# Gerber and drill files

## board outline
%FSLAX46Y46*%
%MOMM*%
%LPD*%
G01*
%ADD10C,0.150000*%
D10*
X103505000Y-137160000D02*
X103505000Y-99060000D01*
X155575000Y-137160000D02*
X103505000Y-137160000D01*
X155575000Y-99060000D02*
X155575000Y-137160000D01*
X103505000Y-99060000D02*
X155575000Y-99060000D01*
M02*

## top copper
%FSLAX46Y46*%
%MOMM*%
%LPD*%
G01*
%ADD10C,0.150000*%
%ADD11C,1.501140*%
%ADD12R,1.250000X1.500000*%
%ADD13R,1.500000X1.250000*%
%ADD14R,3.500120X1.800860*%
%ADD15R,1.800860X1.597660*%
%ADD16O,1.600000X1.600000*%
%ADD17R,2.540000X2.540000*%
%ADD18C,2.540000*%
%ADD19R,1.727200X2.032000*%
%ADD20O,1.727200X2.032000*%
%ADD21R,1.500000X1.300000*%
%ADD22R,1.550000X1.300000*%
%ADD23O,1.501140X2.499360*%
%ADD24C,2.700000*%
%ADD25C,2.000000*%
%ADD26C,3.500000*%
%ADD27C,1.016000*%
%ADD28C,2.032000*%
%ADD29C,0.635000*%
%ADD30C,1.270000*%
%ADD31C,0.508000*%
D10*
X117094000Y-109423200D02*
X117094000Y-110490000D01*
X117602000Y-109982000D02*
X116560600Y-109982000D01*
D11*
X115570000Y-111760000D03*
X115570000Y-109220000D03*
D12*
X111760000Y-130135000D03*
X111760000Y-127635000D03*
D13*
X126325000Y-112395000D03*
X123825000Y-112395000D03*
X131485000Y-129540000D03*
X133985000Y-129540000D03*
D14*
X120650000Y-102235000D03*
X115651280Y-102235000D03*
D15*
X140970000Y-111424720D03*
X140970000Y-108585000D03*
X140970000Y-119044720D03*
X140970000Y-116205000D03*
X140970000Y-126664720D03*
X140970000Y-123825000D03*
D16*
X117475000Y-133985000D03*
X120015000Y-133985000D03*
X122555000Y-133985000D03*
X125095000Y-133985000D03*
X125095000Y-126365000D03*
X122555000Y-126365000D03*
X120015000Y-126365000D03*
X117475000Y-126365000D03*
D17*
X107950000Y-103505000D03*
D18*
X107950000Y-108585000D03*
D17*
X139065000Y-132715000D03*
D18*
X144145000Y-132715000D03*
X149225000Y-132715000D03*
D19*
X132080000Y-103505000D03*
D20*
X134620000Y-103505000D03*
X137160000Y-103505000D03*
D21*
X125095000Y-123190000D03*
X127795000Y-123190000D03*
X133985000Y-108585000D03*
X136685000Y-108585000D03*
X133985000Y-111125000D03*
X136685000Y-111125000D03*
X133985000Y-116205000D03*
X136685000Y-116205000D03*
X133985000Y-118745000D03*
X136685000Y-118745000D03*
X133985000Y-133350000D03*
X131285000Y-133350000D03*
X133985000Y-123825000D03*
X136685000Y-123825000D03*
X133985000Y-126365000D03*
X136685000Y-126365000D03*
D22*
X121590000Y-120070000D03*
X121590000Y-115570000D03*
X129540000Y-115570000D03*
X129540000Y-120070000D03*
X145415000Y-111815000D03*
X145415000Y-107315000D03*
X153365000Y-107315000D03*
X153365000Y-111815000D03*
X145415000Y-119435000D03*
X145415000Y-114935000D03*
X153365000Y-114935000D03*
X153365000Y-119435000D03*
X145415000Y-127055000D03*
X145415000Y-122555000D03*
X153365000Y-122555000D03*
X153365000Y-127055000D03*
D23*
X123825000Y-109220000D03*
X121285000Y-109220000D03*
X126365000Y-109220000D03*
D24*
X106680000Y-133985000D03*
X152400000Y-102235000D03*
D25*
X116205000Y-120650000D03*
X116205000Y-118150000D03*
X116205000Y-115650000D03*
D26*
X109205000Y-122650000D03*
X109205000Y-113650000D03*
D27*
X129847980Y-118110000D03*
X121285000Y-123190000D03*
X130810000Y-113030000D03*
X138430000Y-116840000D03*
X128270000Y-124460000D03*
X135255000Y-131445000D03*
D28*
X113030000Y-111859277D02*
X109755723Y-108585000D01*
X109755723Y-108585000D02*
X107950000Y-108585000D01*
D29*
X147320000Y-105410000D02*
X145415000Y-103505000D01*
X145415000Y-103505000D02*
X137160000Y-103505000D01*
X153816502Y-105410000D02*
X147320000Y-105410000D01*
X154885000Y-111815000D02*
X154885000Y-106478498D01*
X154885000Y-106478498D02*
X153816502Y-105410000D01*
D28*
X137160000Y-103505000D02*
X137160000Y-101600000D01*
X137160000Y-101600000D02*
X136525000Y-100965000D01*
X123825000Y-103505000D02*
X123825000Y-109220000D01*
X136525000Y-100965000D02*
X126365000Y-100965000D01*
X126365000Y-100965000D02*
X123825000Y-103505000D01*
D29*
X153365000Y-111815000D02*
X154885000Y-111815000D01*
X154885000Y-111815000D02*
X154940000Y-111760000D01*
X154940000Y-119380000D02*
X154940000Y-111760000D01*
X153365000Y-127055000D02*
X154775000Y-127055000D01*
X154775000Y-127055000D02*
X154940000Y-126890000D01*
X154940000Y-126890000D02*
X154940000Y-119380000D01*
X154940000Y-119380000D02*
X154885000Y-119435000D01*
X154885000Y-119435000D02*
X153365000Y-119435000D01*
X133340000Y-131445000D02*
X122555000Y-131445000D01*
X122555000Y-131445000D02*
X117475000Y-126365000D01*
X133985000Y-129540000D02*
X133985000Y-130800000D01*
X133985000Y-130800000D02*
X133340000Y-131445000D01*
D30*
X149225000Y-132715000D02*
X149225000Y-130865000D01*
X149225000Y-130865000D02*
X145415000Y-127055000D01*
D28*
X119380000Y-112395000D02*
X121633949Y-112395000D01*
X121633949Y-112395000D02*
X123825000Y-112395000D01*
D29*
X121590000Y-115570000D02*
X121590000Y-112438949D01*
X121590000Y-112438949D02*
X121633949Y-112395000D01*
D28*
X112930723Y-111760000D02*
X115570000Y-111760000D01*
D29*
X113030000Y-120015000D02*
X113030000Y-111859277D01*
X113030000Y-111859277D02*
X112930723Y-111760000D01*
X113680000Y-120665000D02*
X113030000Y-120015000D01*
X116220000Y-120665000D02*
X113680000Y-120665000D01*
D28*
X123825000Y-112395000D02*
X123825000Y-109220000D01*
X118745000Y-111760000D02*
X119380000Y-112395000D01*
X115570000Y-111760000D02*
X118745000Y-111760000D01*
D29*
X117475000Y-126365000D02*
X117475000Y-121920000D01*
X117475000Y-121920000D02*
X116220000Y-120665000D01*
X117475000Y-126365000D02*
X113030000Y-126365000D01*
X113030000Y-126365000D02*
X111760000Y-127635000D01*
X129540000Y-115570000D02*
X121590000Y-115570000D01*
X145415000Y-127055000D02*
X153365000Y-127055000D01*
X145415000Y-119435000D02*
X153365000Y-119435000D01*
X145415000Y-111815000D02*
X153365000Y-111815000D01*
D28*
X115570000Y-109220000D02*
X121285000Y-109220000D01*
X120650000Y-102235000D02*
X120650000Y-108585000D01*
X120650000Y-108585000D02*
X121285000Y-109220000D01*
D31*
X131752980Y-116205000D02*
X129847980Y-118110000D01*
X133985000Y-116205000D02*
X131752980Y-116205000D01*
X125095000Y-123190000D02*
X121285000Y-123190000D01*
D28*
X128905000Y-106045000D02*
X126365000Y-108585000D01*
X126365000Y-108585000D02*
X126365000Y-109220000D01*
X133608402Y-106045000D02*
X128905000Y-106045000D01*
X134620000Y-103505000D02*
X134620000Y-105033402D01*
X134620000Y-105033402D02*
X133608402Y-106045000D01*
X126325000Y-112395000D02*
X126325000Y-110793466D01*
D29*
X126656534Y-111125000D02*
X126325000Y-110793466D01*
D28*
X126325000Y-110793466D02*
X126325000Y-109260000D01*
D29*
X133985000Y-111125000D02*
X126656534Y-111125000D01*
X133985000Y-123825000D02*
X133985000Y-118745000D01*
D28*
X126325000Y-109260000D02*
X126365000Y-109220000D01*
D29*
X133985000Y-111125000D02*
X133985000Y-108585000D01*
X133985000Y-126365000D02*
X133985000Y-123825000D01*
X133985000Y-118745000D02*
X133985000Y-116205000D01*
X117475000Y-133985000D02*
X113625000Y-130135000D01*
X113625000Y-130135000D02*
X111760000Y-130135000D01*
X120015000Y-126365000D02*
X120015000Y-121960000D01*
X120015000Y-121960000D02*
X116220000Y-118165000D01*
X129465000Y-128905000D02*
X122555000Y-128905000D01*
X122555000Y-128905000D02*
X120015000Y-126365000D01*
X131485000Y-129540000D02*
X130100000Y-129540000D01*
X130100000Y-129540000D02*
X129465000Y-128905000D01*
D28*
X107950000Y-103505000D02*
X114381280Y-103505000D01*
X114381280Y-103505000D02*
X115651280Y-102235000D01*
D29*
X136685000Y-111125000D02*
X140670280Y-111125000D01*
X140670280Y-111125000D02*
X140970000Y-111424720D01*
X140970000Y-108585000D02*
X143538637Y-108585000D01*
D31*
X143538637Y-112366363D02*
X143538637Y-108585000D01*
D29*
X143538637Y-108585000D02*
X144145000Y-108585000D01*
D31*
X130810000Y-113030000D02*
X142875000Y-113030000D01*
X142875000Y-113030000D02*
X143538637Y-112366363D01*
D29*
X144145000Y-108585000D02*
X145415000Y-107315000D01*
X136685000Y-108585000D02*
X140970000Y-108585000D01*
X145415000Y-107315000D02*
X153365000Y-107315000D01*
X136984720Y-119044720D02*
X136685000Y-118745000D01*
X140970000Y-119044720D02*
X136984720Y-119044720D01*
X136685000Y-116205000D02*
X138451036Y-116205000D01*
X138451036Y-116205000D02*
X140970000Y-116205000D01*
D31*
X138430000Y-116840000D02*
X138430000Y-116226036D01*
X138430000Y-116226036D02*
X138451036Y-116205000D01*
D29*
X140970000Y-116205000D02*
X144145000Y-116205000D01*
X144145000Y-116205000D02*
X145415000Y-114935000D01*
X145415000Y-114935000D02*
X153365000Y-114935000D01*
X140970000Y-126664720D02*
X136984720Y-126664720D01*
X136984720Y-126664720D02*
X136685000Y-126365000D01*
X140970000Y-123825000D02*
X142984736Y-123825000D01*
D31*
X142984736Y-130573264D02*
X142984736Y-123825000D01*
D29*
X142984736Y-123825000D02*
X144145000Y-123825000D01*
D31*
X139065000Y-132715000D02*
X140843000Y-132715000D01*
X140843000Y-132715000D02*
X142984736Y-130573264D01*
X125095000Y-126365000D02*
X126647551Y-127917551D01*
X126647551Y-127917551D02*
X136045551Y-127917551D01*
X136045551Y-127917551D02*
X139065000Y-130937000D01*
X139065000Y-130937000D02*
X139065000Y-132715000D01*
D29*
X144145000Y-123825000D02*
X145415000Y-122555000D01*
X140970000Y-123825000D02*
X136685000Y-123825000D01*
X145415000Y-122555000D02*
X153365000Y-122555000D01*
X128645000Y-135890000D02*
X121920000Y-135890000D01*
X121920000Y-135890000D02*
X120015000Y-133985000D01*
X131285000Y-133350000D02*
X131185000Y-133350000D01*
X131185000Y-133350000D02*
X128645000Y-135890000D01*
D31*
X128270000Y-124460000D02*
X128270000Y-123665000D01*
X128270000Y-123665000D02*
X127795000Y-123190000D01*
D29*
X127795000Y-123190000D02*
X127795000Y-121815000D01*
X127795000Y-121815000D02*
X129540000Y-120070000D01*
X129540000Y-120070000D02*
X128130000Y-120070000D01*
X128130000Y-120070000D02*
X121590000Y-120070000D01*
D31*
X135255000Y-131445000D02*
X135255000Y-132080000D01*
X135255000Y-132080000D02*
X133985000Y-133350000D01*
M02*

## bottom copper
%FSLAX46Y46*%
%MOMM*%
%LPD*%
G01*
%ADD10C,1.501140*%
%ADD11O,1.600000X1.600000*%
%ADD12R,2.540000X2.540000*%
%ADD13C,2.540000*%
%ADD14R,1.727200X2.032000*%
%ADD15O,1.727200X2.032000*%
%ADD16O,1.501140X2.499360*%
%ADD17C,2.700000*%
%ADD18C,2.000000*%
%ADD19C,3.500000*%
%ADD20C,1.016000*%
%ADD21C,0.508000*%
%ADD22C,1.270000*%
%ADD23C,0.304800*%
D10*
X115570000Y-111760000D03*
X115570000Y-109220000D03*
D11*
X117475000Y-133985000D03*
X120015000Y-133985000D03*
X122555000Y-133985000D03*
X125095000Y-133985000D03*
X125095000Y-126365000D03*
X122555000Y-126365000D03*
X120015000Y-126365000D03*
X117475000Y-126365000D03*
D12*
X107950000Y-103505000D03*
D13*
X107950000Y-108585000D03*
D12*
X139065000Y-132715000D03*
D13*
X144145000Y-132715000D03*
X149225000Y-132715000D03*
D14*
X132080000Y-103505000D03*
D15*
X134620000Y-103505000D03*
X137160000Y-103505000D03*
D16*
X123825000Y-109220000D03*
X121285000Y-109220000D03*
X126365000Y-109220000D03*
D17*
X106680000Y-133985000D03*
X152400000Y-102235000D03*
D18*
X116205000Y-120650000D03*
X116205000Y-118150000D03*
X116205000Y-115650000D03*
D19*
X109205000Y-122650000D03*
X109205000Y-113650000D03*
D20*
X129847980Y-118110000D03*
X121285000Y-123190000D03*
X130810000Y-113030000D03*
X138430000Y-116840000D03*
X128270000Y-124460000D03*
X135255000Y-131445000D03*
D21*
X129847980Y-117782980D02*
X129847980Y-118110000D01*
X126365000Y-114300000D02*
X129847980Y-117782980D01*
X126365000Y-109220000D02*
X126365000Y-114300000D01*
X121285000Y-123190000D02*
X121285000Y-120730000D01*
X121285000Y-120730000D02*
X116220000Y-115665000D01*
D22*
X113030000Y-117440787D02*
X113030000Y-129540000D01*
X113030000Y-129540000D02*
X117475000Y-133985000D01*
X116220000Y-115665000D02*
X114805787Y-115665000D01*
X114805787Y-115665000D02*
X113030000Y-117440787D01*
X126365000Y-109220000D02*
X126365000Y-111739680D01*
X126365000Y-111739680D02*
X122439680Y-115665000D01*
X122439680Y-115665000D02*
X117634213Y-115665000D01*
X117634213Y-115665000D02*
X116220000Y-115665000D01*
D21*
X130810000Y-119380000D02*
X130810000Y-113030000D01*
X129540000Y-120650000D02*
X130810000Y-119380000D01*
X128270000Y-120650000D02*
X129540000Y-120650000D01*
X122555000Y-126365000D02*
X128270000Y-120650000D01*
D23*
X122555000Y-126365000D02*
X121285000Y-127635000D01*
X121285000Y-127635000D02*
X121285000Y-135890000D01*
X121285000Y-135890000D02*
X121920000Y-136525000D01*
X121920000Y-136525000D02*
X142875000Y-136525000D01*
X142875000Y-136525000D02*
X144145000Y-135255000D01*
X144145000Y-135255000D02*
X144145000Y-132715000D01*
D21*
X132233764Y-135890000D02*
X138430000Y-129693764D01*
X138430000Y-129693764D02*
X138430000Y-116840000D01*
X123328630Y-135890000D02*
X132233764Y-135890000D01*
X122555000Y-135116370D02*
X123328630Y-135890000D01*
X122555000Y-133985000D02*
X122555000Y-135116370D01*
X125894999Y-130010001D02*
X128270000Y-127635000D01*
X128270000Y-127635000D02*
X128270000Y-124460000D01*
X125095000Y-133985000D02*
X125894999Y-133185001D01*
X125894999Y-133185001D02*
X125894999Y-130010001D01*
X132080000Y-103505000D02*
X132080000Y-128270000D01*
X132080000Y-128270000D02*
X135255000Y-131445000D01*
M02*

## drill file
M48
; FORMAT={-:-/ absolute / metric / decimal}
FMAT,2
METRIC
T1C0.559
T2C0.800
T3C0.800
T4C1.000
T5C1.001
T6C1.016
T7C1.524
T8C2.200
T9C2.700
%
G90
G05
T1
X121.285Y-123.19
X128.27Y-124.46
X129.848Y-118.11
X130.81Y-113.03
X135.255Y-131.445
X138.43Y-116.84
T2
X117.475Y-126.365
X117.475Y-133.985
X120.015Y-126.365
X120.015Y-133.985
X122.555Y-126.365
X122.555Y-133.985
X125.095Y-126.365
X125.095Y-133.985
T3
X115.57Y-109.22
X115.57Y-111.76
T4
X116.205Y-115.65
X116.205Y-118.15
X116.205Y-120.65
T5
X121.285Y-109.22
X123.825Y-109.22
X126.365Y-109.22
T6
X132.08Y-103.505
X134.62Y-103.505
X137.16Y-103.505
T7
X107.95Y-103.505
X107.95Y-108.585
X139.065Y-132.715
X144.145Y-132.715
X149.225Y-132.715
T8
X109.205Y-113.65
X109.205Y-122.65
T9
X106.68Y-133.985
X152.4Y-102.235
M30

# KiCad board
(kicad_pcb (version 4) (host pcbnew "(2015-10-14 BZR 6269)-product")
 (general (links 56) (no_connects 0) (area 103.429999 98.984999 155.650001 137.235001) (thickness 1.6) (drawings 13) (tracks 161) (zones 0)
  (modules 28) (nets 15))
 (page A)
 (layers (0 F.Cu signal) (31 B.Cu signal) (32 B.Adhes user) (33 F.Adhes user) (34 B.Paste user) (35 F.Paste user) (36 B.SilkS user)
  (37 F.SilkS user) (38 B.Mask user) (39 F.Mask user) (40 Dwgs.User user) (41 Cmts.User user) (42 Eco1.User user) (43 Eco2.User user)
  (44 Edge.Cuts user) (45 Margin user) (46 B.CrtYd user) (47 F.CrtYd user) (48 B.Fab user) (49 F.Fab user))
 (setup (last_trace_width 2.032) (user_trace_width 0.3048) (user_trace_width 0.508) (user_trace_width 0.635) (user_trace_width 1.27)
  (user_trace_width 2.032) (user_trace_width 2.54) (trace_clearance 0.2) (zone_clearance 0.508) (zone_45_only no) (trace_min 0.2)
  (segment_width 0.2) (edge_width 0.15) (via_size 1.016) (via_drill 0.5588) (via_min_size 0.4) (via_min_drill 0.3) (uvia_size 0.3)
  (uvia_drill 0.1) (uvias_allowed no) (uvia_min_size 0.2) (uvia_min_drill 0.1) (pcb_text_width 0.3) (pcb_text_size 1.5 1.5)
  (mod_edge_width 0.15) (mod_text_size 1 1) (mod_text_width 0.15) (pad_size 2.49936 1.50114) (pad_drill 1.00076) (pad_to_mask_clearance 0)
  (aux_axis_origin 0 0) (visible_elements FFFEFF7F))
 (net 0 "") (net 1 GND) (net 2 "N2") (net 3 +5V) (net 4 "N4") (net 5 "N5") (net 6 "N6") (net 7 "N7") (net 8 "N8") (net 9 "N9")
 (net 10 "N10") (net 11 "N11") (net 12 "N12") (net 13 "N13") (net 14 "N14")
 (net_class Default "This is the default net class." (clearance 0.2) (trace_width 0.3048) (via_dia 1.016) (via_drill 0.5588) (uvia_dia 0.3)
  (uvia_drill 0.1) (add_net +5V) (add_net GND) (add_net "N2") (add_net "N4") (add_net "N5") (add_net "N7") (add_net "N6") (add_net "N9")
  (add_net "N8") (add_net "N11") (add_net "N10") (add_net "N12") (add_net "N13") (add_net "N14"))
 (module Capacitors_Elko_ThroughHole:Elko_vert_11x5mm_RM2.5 (layer F.Cu) (at 115.57 109.22 270)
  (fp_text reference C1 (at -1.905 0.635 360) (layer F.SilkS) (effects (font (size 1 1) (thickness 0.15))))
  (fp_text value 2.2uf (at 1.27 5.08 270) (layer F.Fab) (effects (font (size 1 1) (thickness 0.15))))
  (fp_line (start 0.2032 -1.524) (end 1.27 -1.524) (layer F.Cu) (width 0.15))
  (fp_line (start 0.762 -2.032) (end 0.762 -0.9906) (layer F.Cu) (width 0.15))
  (pad 2 thru_hole circle (at 2.54 0 270) (size 1.50114 1.50114) (drill 0.8001) (layers *.Cu *.Mask F.SilkS) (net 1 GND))
  (pad 1 thru_hole circle (at 0 0 270) (size 1.50114 1.50114) (drill 0.8001) (layers *.Cu *.Mask F.SilkS) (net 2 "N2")))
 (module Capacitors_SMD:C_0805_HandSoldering (layer F.Cu) (at 111.76 128.885 90)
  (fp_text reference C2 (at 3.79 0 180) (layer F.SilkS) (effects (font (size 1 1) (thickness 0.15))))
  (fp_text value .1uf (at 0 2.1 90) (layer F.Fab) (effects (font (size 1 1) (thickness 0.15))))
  (pad 1 smd rect (at -1.25 0 90) (size 1.5 1.25) (layers F.Cu F.Paste F.Mask) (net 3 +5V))
  (pad 2 smd rect (at 1.25 0 90) (size 1.5 1.25) (layers F.Cu F.Paste F.Mask) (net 1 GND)))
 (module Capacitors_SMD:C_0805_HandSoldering (layer F.Cu) (at 125.075 112.395 180)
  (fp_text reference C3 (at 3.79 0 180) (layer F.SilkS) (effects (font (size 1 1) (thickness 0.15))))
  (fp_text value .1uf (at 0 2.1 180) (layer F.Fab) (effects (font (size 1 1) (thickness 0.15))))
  (pad 1 smd rect (at -1.25 0 180) (size 1.5 1.25) (layers F.Cu F.Paste F.Mask) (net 3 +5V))
  (pad 2 smd rect (at 1.25 0 180) (size 1.5 1.25) (layers F.Cu F.Paste F.Mask) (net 1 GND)))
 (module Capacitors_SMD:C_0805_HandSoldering (layer F.Cu) (at 132.735 129.54)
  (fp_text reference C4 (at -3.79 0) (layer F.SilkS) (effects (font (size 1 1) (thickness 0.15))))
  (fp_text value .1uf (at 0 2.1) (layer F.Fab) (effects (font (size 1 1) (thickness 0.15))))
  (pad 1 smd rect (at -1.25 0) (size 1.5 1.25) (layers F.Cu F.Paste F.Mask) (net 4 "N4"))
  (pad 2 smd rect (at 1.25 0) (size 1.5 1.25) (layers F.Cu F.Paste F.Mask) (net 1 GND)))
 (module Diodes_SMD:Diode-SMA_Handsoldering (layer F.Cu) (at 118.15064 102.235 180)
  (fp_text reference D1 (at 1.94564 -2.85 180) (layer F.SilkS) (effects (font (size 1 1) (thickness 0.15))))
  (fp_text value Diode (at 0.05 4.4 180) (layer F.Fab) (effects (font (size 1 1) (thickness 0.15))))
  (pad 1 smd rect (at -2.49936 0 180) (size 3.50012 1.80086) (layers F.Cu F.Paste F.Mask) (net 2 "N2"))
  (pad 2 smd rect (at 2.49936 0 180) (size 3.50012 1.80086) (layers F.Cu F.Paste F.Mask) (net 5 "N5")))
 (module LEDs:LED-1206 (layer F.Cu) (at 140.97 110.00486 270)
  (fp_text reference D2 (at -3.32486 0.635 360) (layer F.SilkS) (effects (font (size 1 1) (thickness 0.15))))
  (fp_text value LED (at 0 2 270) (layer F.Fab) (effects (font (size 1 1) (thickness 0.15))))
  (pad 2 smd rect (at 1.41986 0 90) (size 1.59766 1.80086) (layers F.Cu F.Paste F.Mask) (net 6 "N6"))
  (pad 1 smd rect (at -1.41986 0 90) (size 1.59766 1.80086) (layers F.Cu F.Paste F.Mask) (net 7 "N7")))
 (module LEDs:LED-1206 (layer F.Cu) (at 140.97 117.62486 270)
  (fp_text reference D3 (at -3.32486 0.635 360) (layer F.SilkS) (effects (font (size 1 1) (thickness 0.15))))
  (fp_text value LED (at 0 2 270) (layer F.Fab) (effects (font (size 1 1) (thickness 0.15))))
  (pad 2 smd rect (at 1.41986 0 90) (size 1.59766 1.80086) (layers F.Cu F.Paste F.Mask) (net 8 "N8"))
  (pad 1 smd rect (at -1.41986 0 90) (size 1.59766 1.80086) (layers F.Cu F.Paste F.Mask) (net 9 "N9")))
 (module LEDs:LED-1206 (layer F.Cu) (at 140.97 125.24486 270)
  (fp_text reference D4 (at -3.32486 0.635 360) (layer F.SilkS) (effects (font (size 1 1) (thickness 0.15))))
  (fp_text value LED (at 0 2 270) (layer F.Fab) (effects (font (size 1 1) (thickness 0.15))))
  (pad 2 smd rect (at 1.41986 0 90) (size 1.59766 1.80086) (layers F.Cu F.Paste F.Mask) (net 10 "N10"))
  (pad 1 smd rect (at -1.41986 0 90) (size 1.59766 1.80086) (layers F.Cu F.Paste F.Mask) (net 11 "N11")))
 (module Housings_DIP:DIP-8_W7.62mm (layer F.Cu) (at 117.475 133.985 90)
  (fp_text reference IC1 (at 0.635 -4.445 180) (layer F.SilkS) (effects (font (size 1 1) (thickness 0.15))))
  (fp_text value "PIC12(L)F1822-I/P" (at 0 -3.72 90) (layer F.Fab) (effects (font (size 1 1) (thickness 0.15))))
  (pad 1 thru_hole oval (at 0 0 90) (size 1.6 1.6) (drill 0.8) (layers *.Cu *.Mask F.SilkS) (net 3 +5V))
  (pad 2 thru_hole oval (at 0 2.54 90) (size 1.6 1.6) (drill 0.8) (layers *.Cu *.Mask F.SilkS) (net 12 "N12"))
  (pad 3 thru_hole oval (at 0 5.08 90) (size 1.6 1.6) (drill 0.8) (layers *.Cu *.Mask F.SilkS) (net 9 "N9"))
  (pad 4 thru_hole oval (at 0 7.62 90) (size 1.6 1.6) (drill 0.8) (layers *.Cu *.Mask F.SilkS) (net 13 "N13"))
  (pad 5 thru_hole oval (at 7.62 7.62 90) (size 1.6 1.6) (drill 0.8) (layers *.Cu *.Mask F.SilkS) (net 11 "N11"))
  (pad 6 thru_hole oval (at 7.62 5.08 90) (size 1.6 1.6) (drill 0.8) (layers *.Cu *.Mask F.SilkS) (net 7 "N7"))
  (pad 7 thru_hole oval (at 7.62 2.54 90) (size 1.6 1.6) (drill 0.8) (layers *.Cu *.Mask F.SilkS) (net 4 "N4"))
  (pad 8 thru_hole oval (at 7.62 0 90) (size 1.6 1.6) (drill 0.8) (layers *.Cu *.Mask F.SilkS) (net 1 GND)))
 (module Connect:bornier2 (layer F.Cu) (at 107.95 106.045 270)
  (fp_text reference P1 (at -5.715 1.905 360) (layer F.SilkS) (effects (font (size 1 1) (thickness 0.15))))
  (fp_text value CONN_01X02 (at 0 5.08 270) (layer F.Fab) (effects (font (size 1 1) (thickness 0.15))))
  (pad 1 thru_hole rect (at -2.54 0 270) (size 2.54 2.54) (drill 1.524) (layers *.Cu *.Mask F.SilkS) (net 5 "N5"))
  (pad 2 thru_hole circle (at 2.54 0 270) (size 2.54 2.54) (drill 1.524) (layers *.Cu *.Mask F.SilkS) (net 1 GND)))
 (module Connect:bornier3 (layer F.Cu) (at 144.145 132.715)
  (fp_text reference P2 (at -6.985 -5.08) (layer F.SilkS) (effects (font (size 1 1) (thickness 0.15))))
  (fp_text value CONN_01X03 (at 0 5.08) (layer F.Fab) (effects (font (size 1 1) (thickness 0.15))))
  (pad 1 thru_hole rect (at -5.08 0) (size 2.54 2.54) (drill 1.524) (layers *.Cu *.Mask F.SilkS) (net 11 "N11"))
  (pad 2 thru_hole circle (at 0 0) (size 2.54 2.54) (drill 1.524) (layers *.Cu *.Mask F.SilkS) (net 7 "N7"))
  (pad 3 thru_hole circle (at 5.08 0) (size 2.54 2.54) (drill 1.524) (layers *.Cu *.Mask F.SilkS) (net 1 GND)))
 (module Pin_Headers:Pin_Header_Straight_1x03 (layer F.Cu) (at 132.08 103.505 90)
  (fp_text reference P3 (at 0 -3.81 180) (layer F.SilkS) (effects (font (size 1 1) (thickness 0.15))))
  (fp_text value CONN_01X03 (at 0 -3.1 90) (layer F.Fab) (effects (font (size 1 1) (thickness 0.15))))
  (pad 1 thru_hole rect (at 0 0 90) (size 2.032 1.7272) (drill 1.016) (layers *.Cu *.Mask F.SilkS) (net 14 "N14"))
  (pad 2 thru_hole oval (at 0 2.54 90) (size 2.032 1.7272) (drill 1.016) (layers *.Cu *.Mask F.SilkS) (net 3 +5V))
  (pad 3 thru_hole oval (at 0 5.08 90) (size 2.032 1.7272) (drill 1.016) (layers *.Cu *.Mask F.SilkS) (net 1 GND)))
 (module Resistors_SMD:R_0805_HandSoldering (layer F.Cu) (at 126.445 123.19)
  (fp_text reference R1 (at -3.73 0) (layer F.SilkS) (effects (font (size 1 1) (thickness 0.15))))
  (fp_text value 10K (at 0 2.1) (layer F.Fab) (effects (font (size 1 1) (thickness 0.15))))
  (pad 1 smd rect (at -1.35 0) (size 1.5 1.3) (layers F.Cu F.Paste F.Mask) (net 3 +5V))
  (pad 2 smd rect (at 1.35 0) (size 1.5 1.3) (layers F.Cu F.Paste F.Mask) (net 13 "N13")))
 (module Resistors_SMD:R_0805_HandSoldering (layer F.Cu) (at 135.335 108.585)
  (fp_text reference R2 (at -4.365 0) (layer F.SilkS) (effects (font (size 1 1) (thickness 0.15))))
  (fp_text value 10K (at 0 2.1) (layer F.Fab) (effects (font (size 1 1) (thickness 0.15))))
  (pad 1 smd rect (at -1.35 0) (size 1.5 1.3) (layers F.Cu F.Paste F.Mask) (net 3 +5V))
  (pad 2 smd rect (at 1.35 0) (size 1.5 1.3) (layers F.Cu F.Paste F.Mask) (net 7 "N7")))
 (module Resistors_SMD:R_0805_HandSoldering (layer F.Cu) (at 135.335 111.125)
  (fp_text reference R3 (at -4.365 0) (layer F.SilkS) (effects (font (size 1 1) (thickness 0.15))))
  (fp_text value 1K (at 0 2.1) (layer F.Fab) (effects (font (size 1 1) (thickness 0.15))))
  (pad 1 smd rect (at -1.35 0) (size 1.5 1.3) (layers F.Cu F.Paste F.Mask) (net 3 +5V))
  (pad 2 smd rect (at 1.35 0) (size 1.5 1.3) (layers F.Cu F.Paste F.Mask) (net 6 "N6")))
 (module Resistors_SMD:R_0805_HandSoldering (layer F.Cu) (at 135.335 116.205)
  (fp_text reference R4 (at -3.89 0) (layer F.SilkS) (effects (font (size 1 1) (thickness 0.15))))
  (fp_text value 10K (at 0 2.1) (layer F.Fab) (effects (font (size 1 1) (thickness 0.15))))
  (pad 1 smd rect (at -1.35 0) (size 1.5 1.3) (layers F.Cu F.Paste F.Mask) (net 3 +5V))
  (pad 2 smd rect (at 1.35 0) (size 1.5 1.3) (layers F.Cu F.Paste F.Mask) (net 9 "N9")))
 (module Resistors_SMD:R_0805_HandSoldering (layer F.Cu) (at 135.335 118.745)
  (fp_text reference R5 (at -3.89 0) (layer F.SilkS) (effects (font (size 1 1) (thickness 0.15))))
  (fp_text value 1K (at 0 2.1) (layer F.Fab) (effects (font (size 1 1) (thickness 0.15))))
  (pad 1 smd rect (at -1.35 0) (size 1.5 1.3) (layers F.Cu F.Paste F.Mask) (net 3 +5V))
  (pad 2 smd rect (at 1.35 0) (size 1.5 1.3) (layers F.Cu F.Paste F.Mask) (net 8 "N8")))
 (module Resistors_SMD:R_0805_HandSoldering (layer F.Cu) (at 132.635 133.35 180)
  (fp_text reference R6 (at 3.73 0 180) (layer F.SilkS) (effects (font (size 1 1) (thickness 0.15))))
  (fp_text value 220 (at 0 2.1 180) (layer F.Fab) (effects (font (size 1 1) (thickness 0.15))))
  (pad 1 smd rect (at -1.35 0 180) (size 1.5 1.3) (layers F.Cu F.Paste F.Mask) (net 14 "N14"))
  (pad 2 smd rect (at 1.35 0 180) (size 1.5 1.3) (layers F.Cu F.Paste F.Mask) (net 12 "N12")))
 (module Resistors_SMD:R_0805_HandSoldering (layer F.Cu) (at 135.335 123.825)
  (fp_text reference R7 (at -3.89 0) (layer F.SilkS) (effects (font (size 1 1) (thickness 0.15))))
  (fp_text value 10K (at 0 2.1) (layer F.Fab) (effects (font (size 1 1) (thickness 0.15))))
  (pad 1 smd rect (at -1.35 0) (size 1.5 1.3) (layers F.Cu F.Paste F.Mask) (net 3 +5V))
  (pad 2 smd rect (at 1.35 0) (size 1.5 1.3) (layers F.Cu F.Paste F.Mask) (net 11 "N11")))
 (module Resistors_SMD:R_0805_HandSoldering (layer F.Cu) (at 135.335 126.365)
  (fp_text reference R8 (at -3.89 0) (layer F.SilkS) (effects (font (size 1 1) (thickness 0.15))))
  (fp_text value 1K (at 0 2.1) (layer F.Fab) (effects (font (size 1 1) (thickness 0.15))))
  (pad 1 smd rect (at -1.35 0) (size 1.5 1.3) (layers F.Cu F.Paste F.Mask) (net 3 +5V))
  (pad 2 smd rect (at 1.35 0) (size 1.5 1.3) (layers F.Cu F.Paste F.Mask) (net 10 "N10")))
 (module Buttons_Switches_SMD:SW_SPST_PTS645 (layer F.Cu) (at 125.565 117.82)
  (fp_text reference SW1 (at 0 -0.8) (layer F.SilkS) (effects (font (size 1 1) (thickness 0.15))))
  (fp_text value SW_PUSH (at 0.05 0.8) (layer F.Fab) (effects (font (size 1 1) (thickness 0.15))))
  (pad 2 smd rect (at -3.975 2.25) (size 1.55 1.3) (layers F.Cu F.Paste F.Mask) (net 13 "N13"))
  (pad 1 smd rect (at -3.975 -2.25) (size 1.55 1.3) (layers F.Cu F.Paste F.Mask) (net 1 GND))
  (pad 1 smd rect (at 3.975 -2.25) (size 1.55 1.3) (layers F.Cu F.Paste F.Mask) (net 1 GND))
  (pad 2 smd rect (at 3.975 2.25) (size 1.55 1.3) (layers F.Cu F.Paste F.Mask) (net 13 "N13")))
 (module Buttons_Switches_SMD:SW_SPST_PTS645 (layer F.Cu) (at 149.39 109.565)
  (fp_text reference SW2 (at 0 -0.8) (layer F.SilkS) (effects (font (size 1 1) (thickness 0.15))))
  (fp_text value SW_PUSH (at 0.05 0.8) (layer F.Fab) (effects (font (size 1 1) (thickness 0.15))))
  (pad 2 smd rect (at -3.975 2.25) (size 1.55 1.3) (layers F.Cu F.Paste F.Mask) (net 1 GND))
  (pad 1 smd rect (at -3.975 -2.25) (size 1.55 1.3) (layers F.Cu F.Paste F.Mask) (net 7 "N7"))
  (pad 1 smd rect (at 3.975 -2.25) (size 1.55 1.3) (layers F.Cu F.Paste F.Mask) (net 7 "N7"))
  (pad 2 smd rect (at 3.975 2.25) (size 1.55 1.3) (layers F.Cu F.Paste F.Mask) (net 1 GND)))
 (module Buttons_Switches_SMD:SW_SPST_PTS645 (layer F.Cu) (at 149.39 117.185)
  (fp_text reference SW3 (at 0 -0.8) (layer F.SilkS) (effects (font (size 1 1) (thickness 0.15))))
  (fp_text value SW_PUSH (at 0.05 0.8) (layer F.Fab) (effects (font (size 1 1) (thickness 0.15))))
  (pad 2 smd rect (at -3.975 2.25) (size 1.55 1.3) (layers F.Cu F.Paste F.Mask) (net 1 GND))
  (pad 1 smd rect (at -3.975 -2.25) (size 1.55 1.3) (layers F.Cu F.Paste F.Mask) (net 9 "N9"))
  (pad 1 smd rect (at 3.975 -2.25) (size 1.55 1.3) (layers F.Cu F.Paste F.Mask) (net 9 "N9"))
  (pad 2 smd rect (at 3.975 2.25) (size 1.55 1.3) (layers F.Cu F.Paste F.Mask) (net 1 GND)))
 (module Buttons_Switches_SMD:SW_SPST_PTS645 (layer F.Cu) (at 149.39 124.805)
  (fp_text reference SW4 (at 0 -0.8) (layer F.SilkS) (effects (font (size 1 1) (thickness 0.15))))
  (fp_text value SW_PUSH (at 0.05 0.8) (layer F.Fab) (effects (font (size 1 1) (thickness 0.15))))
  (pad 2 smd rect (at -3.975 2.25) (size 1.55 1.3) (layers F.Cu F.Paste F.Mask) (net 1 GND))
  (pad 1 smd rect (at -3.975 -2.25) (size 1.55 1.3) (layers F.Cu F.Paste F.Mask) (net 11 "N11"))
  (pad 1 smd rect (at 3.975 -2.25) (size 1.55 1.3) (layers F.Cu F.Paste F.Mask) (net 11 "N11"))
  (pad 2 smd rect (at 3.975 2.25) (size 1.55 1.3) (layers F.Cu F.Paste F.Mask) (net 1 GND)))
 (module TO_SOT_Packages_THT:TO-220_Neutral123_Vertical (layer F.Cu) (at 123.825 109.22)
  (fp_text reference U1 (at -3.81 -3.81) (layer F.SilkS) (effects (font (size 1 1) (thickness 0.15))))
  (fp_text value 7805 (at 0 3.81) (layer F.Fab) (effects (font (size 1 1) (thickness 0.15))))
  (pad GND thru_hole oval (at 0 0 90) (size 2.49936 1.50114) (drill 1.00076) (layers *.Cu *.Mask F.SilkS) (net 1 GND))
  (pad VI thru_hole oval (at -2.54 0 90) (size 2.49936 1.50114) (drill 1.00076) (layers *.Cu *.Mask F.SilkS) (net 2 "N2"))
  (pad VO thru_hole oval (at 2.54 0 90) (size 2.49936 1.50114) (drill 1.00076) (layers *.Cu *.Mask F.SilkS) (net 3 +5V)))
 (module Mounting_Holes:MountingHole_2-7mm (layer F.Cu) (at 106.68 133.985)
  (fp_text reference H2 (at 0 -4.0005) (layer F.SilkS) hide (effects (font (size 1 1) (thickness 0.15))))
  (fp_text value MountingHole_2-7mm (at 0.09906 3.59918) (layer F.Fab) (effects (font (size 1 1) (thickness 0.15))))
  (pad 1 thru_hole circle (at 0 0) (size 2.7 2.7) (drill 2.7) (layers)))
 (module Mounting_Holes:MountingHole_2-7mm (layer F.Cu) (at 152.4 102.235)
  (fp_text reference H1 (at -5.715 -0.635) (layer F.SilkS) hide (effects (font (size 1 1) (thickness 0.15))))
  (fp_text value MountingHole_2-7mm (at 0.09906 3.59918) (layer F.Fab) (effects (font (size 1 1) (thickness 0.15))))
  (pad 1 thru_hole circle (at 0 0) (size 2.7 2.7) (drill 2.7) (layers)))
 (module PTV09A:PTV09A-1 (layer F.Cu) (at 116.205 118.15 90)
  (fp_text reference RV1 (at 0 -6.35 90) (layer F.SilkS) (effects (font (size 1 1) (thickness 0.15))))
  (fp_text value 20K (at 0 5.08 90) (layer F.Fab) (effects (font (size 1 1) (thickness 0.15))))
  (pad 1 thru_hole circle (at -2.5 0 90) (size 2 2) (drill 1) (layers *.Cu *.Mask F.SilkS) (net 1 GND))
  (pad 2 thru_hole circle (at 0 0 90) (size 2 2) (drill 1) (layers *.Cu *.Mask F.SilkS) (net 4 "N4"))
  (pad 3 thru_hole circle (at 2.5 0 90) (size 2 2) (drill 1) (layers *.Cu *.Mask F.SilkS) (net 3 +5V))
  (pad 4 thru_hole circle (at -4.5 -7 90) (size 3.5 3.5) (drill 2.2) (layers *.Cu *.Mask F.SilkS))
  (pad 4 thru_hole circle (at 4.5 -7 90) (size 3.5 3.5) (drill 2.2) (layers *.Cu *.Mask F.SilkS)))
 (gr_line (start 103.505 137.16) (end 103.505 99.06) (layer Edge.Cuts) (width 0.15))
 (gr_line (start 155.575 137.16) (end 103.505 137.16) (layer Edge.Cuts) (width 0.15))
 (gr_line (start 155.575 99.06) (end 155.575 137.16) (layer Edge.Cuts) (width 0.15))
 (gr_line (start 103.505 99.06) (end 155.575 99.06) (layer Edge.Cuts) (width 0.15))
 (segment (start 113.03 111.859277) (end 109.755723 108.585) (width 2.032) (layer F.Cu) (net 1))
 (segment (start 109.755723 108.585) (end 107.95 108.585) (width 2.032) (layer F.Cu) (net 1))
 (segment (start 147.32 105.41) (end 145.415 103.505) (width 0.635) (layer F.Cu) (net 1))
 (segment (start 145.415 103.505) (end 137.16 103.505) (width 0.635) (layer F.Cu) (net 1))
 (segment (start 153.816502 105.41) (end 147.32 105.41) (width 0.635) (layer F.Cu) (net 1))
 (segment (start 154.885 111.815) (end 154.885 106.478498) (width 0.635) (layer F.Cu) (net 1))
 (segment (start 154.885 106.478498) (end 153.816502 105.41) (width 0.635) (layer F.Cu) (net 1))
 (segment (start 137.16 103.505) (end 137.16 101.6) (width 2.032) (layer F.Cu) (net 1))
 (segment (start 137.16 101.6) (end 136.525 100.965) (width 2.032) (layer F.Cu) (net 1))
 (segment (start 123.825 103.505) (end 123.825 109.22) (width 2.032) (layer F.Cu) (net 1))
 (segment (start 136.525 100.965) (end 126.365 100.965) (width 2.032) (layer F.Cu) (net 1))
 (segment (start 126.365 100.965) (end 123.825 103.505) (width 2.032) (layer F.Cu) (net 1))
 (segment (start 153.365 111.815) (end 154.885 111.815) (width 0.635) (layer F.Cu) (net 1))
 (segment (start 154.885 111.815) (end 154.94 111.76) (width 0.635) (layer F.Cu) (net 1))
 (segment (start 154.94 119.38) (end 154.94 111.76) (width 0.635) (layer F.Cu) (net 1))
 (segment (start 153.365 127.055) (end 154.775 127.055) (width 0.635) (layer F.Cu) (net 1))
 (segment (start 154.775 127.055) (end 154.94 126.89) (width 0.635) (layer F.Cu) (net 1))
 (segment (start 154.94 126.89) (end 154.94 119.38) (width 0.635) (layer F.Cu) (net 1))
 (segment (start 154.94 119.38) (end 154.885 119.435) (width 0.635) (layer F.Cu) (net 1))
 (segment (start 154.885 119.435) (end 153.365 119.435) (width 0.635) (layer F.Cu) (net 1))
 (segment (start 133.34 131.445) (end 122.555 131.445) (width 0.635) (layer F.Cu) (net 1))
 (segment (start 122.555 131.445) (end 117.475 126.365) (width 0.635) (layer F.Cu) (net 1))
 (segment (start 133.985 129.54) (end 133.985 130.8) (width 0.635) (layer F.Cu) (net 1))
 (segment (start 133.985 130.8) (end 133.34 131.445) (width 0.635) (layer F.Cu) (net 1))
 (segment (start 149.225 132.715) (end 149.225 130.865) (width 1.27) (layer F.Cu) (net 1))
 (segment (start 149.225 130.865) (end 145.415 127.055) (width 1.27) (layer F.Cu) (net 1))
 (segment (start 119.38 112.395) (end 121.633949 112.395) (width 2.032) (layer F.Cu) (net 1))
 (segment (start 121.633949 112.395) (end 123.825 112.395) (width 2.032) (layer F.Cu) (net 1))
 (segment (start 121.59 115.57) (end 121.59 112.438949) (width 0.635) (layer F.Cu) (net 1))
 (segment (start 121.59 112.438949) (end 121.633949 112.395) (width 0.635) (layer F.Cu) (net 1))
 (segment (start 112.930723 111.76) (end 115.57 111.76) (width 2.032) (layer F.Cu) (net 1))
 (segment (start 113.03 120.015) (end 113.03 111.859277) (width 0.635) (layer F.Cu) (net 1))
 (segment (start 113.03 111.859277) (end 112.930723 111.76) (width 0.635) (layer F.Cu) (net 1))
 (segment (start 113.68 120.665) (end 113.03 120.015) (width 0.635) (layer F.Cu) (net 1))
 (segment (start 116.22 120.665) (end 113.68 120.665) (width 0.635) (layer F.Cu) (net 1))
 (segment (start 123.825 112.395) (end 123.825 109.22) (width 2.032) (layer F.Cu) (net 1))
 (segment (start 118.745 111.76) (end 119.38 112.395) (width 2.032) (layer F.Cu) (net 1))
 (segment (start 115.57 111.76) (end 118.745 111.76) (width 2.032) (layer F.Cu) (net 1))
 (segment (start 117.475 126.365) (end 117.475 121.92) (width 0.635) (layer F.Cu) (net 1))
 (segment (start 117.475 121.92) (end 116.22 120.665) (width 0.635) (layer F.Cu) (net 1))
 (segment (start 117.475 126.365) (end 113.03 126.365) (width 0.635) (layer F.Cu) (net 1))
 (segment (start 113.03 126.365) (end 111.76 127.635) (width 0.635) (layer F.Cu) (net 1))
 (segment (start 129.54 115.57) (end 121.59 115.57) (width 0.635) (layer F.Cu) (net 1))
 (segment (start 145.415 127.055) (end 153.365 127.055) (width 0.635) (layer F.Cu) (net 1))
 (segment (start 145.415 119.435) (end 153.365 119.435) (width 0.635) (layer F.Cu) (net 1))
 (segment (start 145.415 111.815) (end 153.365 111.815) (width 0.635) (layer F.Cu) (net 1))
 (segment (start 115.57 109.22) (end 121.285 109.22) (width 2.032) (layer F.Cu) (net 2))
 (segment (start 120.65 102.235) (end 120.65 108.585) (width 2.032) (layer F.Cu) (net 2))
 (segment (start 120.65 108.585) (end 121.285 109.22) (width 2.032) (layer F.Cu) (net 2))
 (segment (start 129.84798 117.78298) (end 129.84798 118.11) (width 0.508) (layer B.Cu) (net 3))
 (segment (start 126.365 114.3) (end 129.84798 117.78298) (width 0.508) (layer B.Cu) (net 3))
 (segment (start 126.365 109.22) (end 126.365 114.3) (width 0.508) (layer B.Cu) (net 3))
 (via (at 129.84798 118.11) (size 1.016) (drill 0.5588) (layers F.Cu B.Cu) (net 3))
 (segment (start 131.75298 116.205) (end 129.84798 118.11) (width 0.508) (layer F.Cu) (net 3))
 (segment (start 133.985 116.205) (end 131.75298 116.205) (width 0.508) (layer F.Cu) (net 3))
 (segment (start 121.285 123.19) (end 121.285 120.73) (width 0.508) (layer B.Cu) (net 3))
 (segment (start 121.285 120.73) (end 116.22 115.665) (width 0.508) (layer B.Cu) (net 3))
 (segment (start 125.095 123.19) (end 121.285 123.19) (width 0.508) (layer F.Cu) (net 3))
 (via (at 121.285 123.19) (size 1.016) (drill 0.5588) (layers F.Cu B.Cu) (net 3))
 (segment (start 128.905 106.045) (end 126.365 108.585) (width 2.032) (layer F.Cu) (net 3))
 (segment (start 126.365 108.585) (end 126.365 109.22) (width 2.032) (layer F.Cu) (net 3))
 (segment (start 133.608402 106.045) (end 128.905 106.045) (width 2.032) (layer F.Cu) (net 3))
 (segment (start 134.62 103.505) (end 134.62 105.033402) (width 2.032) (layer F.Cu) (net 3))
 (segment (start 134.62 105.033402) (end 133.608402 106.045) (width 2.032) (layer F.Cu) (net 3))
 (segment (start 113.03 117.440787) (end 113.03 129.54) (width 1.27) (layer B.Cu) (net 3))
 (segment (start 113.03 129.54) (end 117.475 133.985) (width 1.27) (layer B.Cu) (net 3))
 (segment (start 116.22 115.665) (end 114.805787 115.665) (width 1.27) (layer B.Cu) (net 3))
 (segment (start 114.805787 115.665) (end 113.03 117.440787) (width 1.27) (layer B.Cu) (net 3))
 (segment (start 126.365 109.22) (end 126.365 111.73968) (width 1.27) (layer B.Cu) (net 3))
 (segment (start 126.365 111.73968) (end 122.43968 115.665) (width 1.27) (layer B.Cu) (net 3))
 (segment (start 122.43968 115.665) (end 117.634213 115.665) (width 1.27) (layer B.Cu) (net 3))
 (segment (start 117.634213 115.665) (end 116.22 115.665) (width 1.27) (layer B.Cu) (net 3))
 (segment (start 126.325 112.395) (end 126.325 110.793466) (width 2.032) (layer F.Cu) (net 3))
 (segment (start 126.656534 111.125) (end 126.325 110.793466) (width 0.635) (layer F.Cu) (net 3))
 (segment (start 126.325 110.793466) (end 126.325 109.26) (width 2.032) (layer F.Cu) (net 3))
 (segment (start 133.985 111.125) (end 126.656534 111.125) (width 0.635) (layer F.Cu) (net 3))
 (segment (start 133.985 123.825) (end 133.985 118.745) (width 0.635) (layer F.Cu) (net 3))
 (segment (start 126.325 109.26) (end 126.365 109.22) (width 2.032) (layer F.Cu) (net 3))
 (segment (start 133.985 111.125) (end 133.985 108.585) (width 0.635) (layer F.Cu) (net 3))
 (segment (start 133.985 126.365) (end 133.985 123.825) (width 0.635) (layer F.Cu) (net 3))
 (segment (start 133.985 118.745) (end 133.985 116.205) (width 0.635) (layer F.Cu) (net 3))
 (segment (start 117.475 133.985) (end 113.625 130.135) (width 0.635) (layer F.Cu) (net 3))
 (segment (start 113.625 130.135) (end 111.76 130.135) (width 0.635) (layer F.Cu) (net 3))
 (segment (start 120.015 126.365) (end 120.015 121.96) (width 0.635) (layer F.Cu) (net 4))
 (segment (start 120.015 121.96) (end 116.22 118.165) (width 0.635) (layer F.Cu) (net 4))
 (segment (start 129.465 128.905) (end 122.555 128.905) (width 0.635) (layer F.Cu) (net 4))
 (segment (start 122.555 128.905) (end 120.015 126.365) (width 0.635) (layer F.Cu) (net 4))
 (segment (start 131.485 129.54) (end 130.1 129.54) (width 0.635) (layer F.Cu) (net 4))
 (segment (start 130.1 129.54) (end 129.465 128.905) (width 0.635) (layer F.Cu) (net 4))
 (segment (start 107.95 103.505) (end 114.38128 103.505) (width 2.032) (layer F.Cu) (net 5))
 (segment (start 114.38128 103.505) (end 115.65128 102.235) (width 2.032) (layer F.Cu) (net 5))
 (segment (start 136.685 111.125) (end 140.67028 111.125) (width 0.635) (layer F.Cu) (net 6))
 (segment (start 140.67028 111.125) (end 140.97 111.42472) (width 0.635) (layer F.Cu) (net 6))
 (segment (start 140.97 108.585) (end 143.538637 108.585) (width 0.635) (layer F.Cu) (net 7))
 (segment (start 143.538637 112.366363) (end 143.538637 108.585) (width 0.508) (layer F.Cu) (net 7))
 (segment (start 143.538637 108.585) (end 144.145 108.585) (width 0.635) (layer F.Cu) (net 7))
 (segment (start 130.81 113.03) (end 142.875 113.03) (width 0.508) (layer F.Cu) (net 7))
 (segment (start 142.875 113.03) (end 143.538637 112.366363) (width 0.508) (layer F.Cu) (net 7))
 (via (at 130.81 113.03) (size 1.016) (drill 0.5588) (layers F.Cu B.Cu) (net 7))
 (segment (start 130.81 119.38) (end 130.81 113.03) (width 0.508) (layer B.Cu) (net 7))
 (segment (start 129.54 120.65) (end 130.81 119.38) (width 0.508) (layer B.Cu) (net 7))
 (segment (start 128.27 120.65) (end 129.54 120.65) (width 0.508) (layer B.Cu) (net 7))
 (segment (start 122.555 126.365) (end 128.27 120.65) (width 0.508) (layer B.Cu) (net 7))
 (segment (start 122.555 126.365) (end 121.285 127.635) (width 0.3048) (layer B.Cu) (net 7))
 (segment (start 121.285 127.635) (end 121.285 135.89) (width 0.3048) (layer B.Cu) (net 7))
 (segment (start 121.285 135.89) (end 121.92 136.525) (width 0.3048) (layer B.Cu) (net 7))
 (segment (start 121.92 136.525) (end 142.875 136.525) (width 0.3048) (layer B.Cu) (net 7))
 (segment (start 142.875 136.525) (end 144.145 135.255) (width 0.3048) (layer B.Cu) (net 7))
 (segment (start 144.145 135.255) (end 144.145 132.715) (width 0.3048) (layer B.Cu) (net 7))
 (segment (start 144.145 108.585) (end 145.415 107.315) (width 0.635) (layer F.Cu) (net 7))
 (segment (start 136.685 108.585) (end 140.97 108.585) (width 0.635) (layer F.Cu) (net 7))
 (segment (start 145.415 107.315) (end 153.365 107.315) (width 0.635) (layer F.Cu) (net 7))
 (segment (start 136.98472 119.04472) (end 136.685 118.745) (width 0.635) (layer F.Cu) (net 8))
 (segment (start 140.97 119.04472) (end 136.98472 119.04472) (width 0.635) (layer F.Cu) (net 8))
 (segment (start 132.233764 135.89) (end 138.43 129.693764) (width 0.508) (layer B.Cu) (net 9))
 (segment (start 138.43 129.693764) (end 138.43 116.84) (width 0.508) (layer B.Cu) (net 9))
 (segment (start 123.32863 135.89) (end 132.233764 135.89) (width 0.508) (layer B.Cu) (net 9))
 (segment (start 122.555 135.11637) (end 123.32863 135.89) (width 0.508) (layer B.Cu) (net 9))
 (segment (start 122.555 133.985) (end 122.555 135.11637) (width 0.508) (layer B.Cu) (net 9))
 (segment (start 136.685 116.205) (end 138.451036 116.205) (width 0.635) (layer F.Cu) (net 9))
 (segment (start 138.451036 116.205) (end 140.97 116.205) (width 0.635) (layer F.Cu) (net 9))
 (segment (start 138.43 116.84) (end 138.43 116.226036) (width 0.508) (layer F.Cu) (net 9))
 (segment (start 138.43 116.226036) (end 138.451036 116.205) (width 0.508) (layer F.Cu) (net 9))
 (via (at 138.43 116.84) (size 1.016) (drill 0.5588) (layers F.Cu B.Cu) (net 9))
 (segment (start 140.97 116.205) (end 144.145 116.205) (width 0.635) (layer F.Cu) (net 9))
 (segment (start 144.145 116.205) (end 145.415 114.935) (width 0.635) (layer F.Cu) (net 9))
 (segment (start 145.415 114.935) (end 153.365 114.935) (width 0.635) (layer F.Cu) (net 9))
 (segment (start 140.97 126.66472) (end 136.98472 126.66472) (width 0.635) (layer F.Cu) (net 10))
 (segment (start 136.98472 126.66472) (end 136.685 126.365) (width 0.635) (layer F.Cu) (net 10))
 (segment (start 140.97 123.825) (end 142.984736 123.825) (width 0.635) (layer F.Cu) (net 11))
 (segment (start 142.984736 130.573264) (end 142.984736 123.825) (width 0.508) (layer F.Cu) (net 11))
 (segment (start 142.984736 123.825) (end 144.145 123.825) (width 0.635) (layer F.Cu) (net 11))
 (segment (start 139.065 132.715) (end 140.843 132.715) (width 0.508) (layer F.Cu) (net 11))
 (segment (start 140.843 132.715) (end 142.984736 130.573264) (width 0.508) (layer F.Cu) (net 11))
 (segment (start 125.095 126.365) (end 126.647551 127.917551) (width 0.508) (layer F.Cu) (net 11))
 (segment (start 126.647551 127.917551) (end 136.045551 127.917551) (width 0.508) (layer F.Cu) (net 11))
 (segment (start 136.045551 127.917551) (end 139.065 130.937) (width 0.508) (layer F.Cu) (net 11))
 (segment (start 139.065 130.937) (end 139.065 132.715) (width 0.508) (layer F.Cu) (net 11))
 (segment (start 144.145 123.825) (end 145.415 122.555) (width 0.635) (layer F.Cu) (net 11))
 (segment (start 140.97 123.825) (end 136.685 123.825) (width 0.635) (layer F.Cu) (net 11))
 (segment (start 145.415 122.555) (end 153.365 122.555) (width 0.635) (layer F.Cu) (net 11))
 (segment (start 128.645 135.89) (end 121.92 135.89) (width 0.635) (layer F.Cu) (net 12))
 (segment (start 121.92 135.89) (end 120.015 133.985) (width 0.635) (layer F.Cu) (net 12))
 (segment (start 131.285 133.35) (end 131.185 133.35) (width 0.635) (layer F.Cu) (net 12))
 (segment (start 131.185 133.35) (end 128.645 135.89) (width 0.635) (layer F.Cu) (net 12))
 (segment (start 128.27 124.46) (end 128.27 123.665) (width 0.508) (layer F.Cu) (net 13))
 (segment (start 128.27 123.665) (end 127.795 123.19) (width 0.508) (layer F.Cu) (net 13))
 (via (at 128.27 124.46) (size 1.016) (drill 0.5588) (layers F.Cu B.Cu) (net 13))
 (segment (start 125.894999 130.010001) (end 128.27 127.635) (width 0.508) (layer B.Cu) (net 13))
 (segment (start 128.27 127.635) (end 128.27 124.46) (width 0.508) (layer B.Cu) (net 13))
 (segment (start 125.095 133.985) (end 125.894999 133.185001) (width 0.508) (layer B.Cu) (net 13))
 (segment (start 125.894999 133.185001) (end 125.894999 130.010001) (width 0.508) (layer B.Cu) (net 13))
 (segment (start 127.795 123.19) (end 127.795 121.815) (width 0.635) (layer F.Cu) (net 13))
 (segment (start 127.795 121.815) (end 129.54 120.07) (width 0.635) (layer F.Cu) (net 13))
 (segment (start 129.54 120.07) (end 128.13 120.07) (width 0.635) (layer F.Cu) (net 13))
 (segment (start 128.13 120.07) (end 121.59 120.07) (width 0.635) (layer F.Cu) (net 13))
 (segment (start 135.255 131.445) (end 135.255 132.08) (width 0.508) (layer F.Cu) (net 14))
 (segment (start 135.255 132.08) (end 133.985 133.35) (width 0.508) (layer F.Cu) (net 14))
 (via (at 135.255 131.445) (size 1.016) (drill 0.5588) (layers F.Cu B.Cu) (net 14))
 (segment (start 132.08 103.505) (end 132.08 128.27) (width 0.508) (layer B.Cu) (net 14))
 (segment (start 132.08 128.27) (end 135.255 131.445) (width 0.508) (layer B.Cu) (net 14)))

